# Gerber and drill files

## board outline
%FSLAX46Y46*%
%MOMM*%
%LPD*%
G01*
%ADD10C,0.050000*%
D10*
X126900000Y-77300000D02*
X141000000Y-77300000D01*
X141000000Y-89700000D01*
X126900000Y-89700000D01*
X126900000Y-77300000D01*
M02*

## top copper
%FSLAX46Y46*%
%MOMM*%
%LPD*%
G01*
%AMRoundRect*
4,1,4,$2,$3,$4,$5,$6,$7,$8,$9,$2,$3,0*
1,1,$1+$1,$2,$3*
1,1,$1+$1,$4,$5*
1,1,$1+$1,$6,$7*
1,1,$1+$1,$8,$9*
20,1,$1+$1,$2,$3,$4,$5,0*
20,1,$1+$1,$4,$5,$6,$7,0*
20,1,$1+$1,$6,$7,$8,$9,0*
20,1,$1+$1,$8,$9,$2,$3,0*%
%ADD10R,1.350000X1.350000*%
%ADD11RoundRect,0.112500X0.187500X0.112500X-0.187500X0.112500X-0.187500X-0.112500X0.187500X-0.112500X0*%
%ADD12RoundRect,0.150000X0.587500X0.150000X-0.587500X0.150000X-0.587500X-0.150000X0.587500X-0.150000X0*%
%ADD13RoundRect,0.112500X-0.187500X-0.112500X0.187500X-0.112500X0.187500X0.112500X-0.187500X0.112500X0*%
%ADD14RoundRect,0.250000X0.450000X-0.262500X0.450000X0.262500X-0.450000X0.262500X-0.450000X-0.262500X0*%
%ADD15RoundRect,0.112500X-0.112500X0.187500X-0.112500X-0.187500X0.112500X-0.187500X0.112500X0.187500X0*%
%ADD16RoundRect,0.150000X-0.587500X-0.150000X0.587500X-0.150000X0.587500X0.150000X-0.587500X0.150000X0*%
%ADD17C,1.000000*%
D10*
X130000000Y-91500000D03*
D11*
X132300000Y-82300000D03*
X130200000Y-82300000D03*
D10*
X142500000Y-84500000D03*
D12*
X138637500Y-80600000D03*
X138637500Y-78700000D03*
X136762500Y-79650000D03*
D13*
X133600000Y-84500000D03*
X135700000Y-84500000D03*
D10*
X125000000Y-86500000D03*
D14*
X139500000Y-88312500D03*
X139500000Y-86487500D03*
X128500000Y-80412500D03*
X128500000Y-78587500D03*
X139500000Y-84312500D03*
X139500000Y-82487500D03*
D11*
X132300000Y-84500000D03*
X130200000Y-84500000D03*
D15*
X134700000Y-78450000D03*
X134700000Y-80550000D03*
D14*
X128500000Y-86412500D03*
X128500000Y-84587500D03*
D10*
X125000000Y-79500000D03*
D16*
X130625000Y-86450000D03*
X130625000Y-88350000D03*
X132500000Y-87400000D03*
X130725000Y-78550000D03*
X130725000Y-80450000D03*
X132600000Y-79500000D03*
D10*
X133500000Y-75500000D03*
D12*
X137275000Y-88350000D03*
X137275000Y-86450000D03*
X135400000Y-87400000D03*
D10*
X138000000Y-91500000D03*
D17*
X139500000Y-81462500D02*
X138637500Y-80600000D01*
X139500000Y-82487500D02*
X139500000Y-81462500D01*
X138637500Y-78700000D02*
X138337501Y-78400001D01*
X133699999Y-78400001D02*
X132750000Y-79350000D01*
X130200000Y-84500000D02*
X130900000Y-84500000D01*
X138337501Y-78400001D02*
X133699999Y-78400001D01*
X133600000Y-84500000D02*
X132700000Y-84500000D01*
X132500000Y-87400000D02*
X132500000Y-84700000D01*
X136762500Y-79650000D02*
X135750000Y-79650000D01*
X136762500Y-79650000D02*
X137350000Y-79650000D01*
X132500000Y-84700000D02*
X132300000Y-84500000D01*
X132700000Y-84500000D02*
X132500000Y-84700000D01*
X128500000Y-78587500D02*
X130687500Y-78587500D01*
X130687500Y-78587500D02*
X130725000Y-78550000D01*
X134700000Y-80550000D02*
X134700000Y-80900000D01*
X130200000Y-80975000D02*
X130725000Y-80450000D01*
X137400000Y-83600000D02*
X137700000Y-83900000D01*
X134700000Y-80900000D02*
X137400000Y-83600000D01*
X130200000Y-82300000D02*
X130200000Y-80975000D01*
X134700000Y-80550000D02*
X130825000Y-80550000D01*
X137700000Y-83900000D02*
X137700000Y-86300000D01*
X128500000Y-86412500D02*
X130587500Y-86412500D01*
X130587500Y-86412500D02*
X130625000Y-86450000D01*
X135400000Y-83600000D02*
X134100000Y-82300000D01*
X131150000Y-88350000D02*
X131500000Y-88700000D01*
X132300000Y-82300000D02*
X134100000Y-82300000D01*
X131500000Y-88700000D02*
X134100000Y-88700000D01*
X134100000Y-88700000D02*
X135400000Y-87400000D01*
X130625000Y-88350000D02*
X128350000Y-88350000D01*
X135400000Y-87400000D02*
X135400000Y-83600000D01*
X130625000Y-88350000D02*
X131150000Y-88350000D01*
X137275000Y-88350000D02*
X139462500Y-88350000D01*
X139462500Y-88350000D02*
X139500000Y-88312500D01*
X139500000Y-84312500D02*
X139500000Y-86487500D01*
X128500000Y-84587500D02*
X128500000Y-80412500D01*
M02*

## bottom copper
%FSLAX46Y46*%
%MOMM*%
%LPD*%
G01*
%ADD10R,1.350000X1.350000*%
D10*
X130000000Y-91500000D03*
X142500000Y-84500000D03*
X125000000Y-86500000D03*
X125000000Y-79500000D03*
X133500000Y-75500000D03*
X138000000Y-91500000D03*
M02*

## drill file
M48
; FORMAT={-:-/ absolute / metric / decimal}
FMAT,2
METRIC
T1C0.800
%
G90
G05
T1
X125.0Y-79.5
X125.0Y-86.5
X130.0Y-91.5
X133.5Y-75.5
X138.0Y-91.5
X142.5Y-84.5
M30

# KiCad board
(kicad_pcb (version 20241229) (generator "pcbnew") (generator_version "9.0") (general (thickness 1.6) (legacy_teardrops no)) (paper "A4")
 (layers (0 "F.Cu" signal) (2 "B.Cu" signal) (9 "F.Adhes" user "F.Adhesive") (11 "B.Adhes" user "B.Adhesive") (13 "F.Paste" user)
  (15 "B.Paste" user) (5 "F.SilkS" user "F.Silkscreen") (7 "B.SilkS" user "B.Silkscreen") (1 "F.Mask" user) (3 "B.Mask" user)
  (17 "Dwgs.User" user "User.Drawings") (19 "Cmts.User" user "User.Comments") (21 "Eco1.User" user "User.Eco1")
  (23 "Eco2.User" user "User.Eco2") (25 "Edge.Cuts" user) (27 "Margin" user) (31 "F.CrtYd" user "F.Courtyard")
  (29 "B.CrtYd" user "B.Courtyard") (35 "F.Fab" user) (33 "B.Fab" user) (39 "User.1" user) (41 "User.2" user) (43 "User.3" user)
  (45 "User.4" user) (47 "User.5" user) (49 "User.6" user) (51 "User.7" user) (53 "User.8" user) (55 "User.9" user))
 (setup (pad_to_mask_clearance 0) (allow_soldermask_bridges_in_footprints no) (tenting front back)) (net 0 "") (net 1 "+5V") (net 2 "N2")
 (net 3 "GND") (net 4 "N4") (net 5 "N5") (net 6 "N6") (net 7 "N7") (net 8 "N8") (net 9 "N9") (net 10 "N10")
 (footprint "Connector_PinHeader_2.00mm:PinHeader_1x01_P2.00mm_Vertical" (layer "F.Cu") (at 130 91.5)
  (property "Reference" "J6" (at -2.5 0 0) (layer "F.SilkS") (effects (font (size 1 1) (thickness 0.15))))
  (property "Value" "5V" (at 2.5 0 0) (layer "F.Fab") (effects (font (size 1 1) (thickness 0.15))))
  (pad "1" thru_hole rect (at 0 0) (size 1.35 1.35) (drill 0.8) (layers "*.Cu" "*.Mask") (remove_unused_layers no) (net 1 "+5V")))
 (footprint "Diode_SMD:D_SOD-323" (layer "F.Cu") (at 131.25 82.3 180)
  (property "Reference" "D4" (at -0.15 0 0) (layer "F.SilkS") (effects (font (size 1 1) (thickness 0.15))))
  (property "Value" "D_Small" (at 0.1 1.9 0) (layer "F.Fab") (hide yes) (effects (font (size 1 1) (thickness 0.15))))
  (pad "1" smd roundrect (at -1.05 0 180) (size 0.6 0.45) (layers "F.Cu" "F.Mask" "F.Paste") (roundrect_rratio 0.25) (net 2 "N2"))
  (pad "2" smd roundrect (at 1.05 0 180) (size 0.6 0.45) (layers "F.Cu" "F.Mask" "F.Paste") (roundrect_rratio 0.25) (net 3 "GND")))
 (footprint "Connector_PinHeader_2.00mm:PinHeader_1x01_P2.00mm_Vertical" (layer "F.Cu") (at 142.5 84.5)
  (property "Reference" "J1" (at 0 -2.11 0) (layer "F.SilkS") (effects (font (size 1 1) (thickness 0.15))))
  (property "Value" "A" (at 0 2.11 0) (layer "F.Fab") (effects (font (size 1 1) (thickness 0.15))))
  (pad "1" thru_hole rect (at 0 0) (size 1.35 1.35) (drill 0.8) (layers "*.Cu" "*.Mask") (remove_unused_layers no) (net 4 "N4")))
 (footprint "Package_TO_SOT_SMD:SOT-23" (layer "F.Cu") (at 137.7 79.65 180)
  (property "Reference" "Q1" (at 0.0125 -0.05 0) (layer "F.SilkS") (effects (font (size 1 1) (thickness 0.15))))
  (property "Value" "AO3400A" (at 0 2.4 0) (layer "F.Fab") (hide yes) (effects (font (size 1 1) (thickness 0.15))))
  (pad "1" smd roundrect (at -0.9375 -0.95 180) (size 1.475 0.6) (layers "F.Cu" "F.Mask" "F.Paste") (roundrect_rratio 0.25) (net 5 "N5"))
  (pad "2" smd roundrect (at -0.9375 0.95 180) (size 1.475 0.6) (layers "F.Cu" "F.Mask" "F.Paste") (roundrect_rratio 0.25) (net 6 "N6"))
  (pad "3" smd roundrect (at 0.9375 0 180) (size 1.475 0.6) (layers "F.Cu" "F.Mask" "F.Paste") (roundrect_rratio 0.25) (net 1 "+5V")))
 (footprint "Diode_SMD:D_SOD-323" (layer "F.Cu") (at 134.65 84.5)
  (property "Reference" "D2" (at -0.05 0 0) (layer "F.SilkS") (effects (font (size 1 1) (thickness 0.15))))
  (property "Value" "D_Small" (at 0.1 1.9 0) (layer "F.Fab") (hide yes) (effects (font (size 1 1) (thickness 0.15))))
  (pad "1" smd roundrect (at -1.05 0) (size 0.6 0.45) (layers "F.Cu" "F.Mask" "F.Paste") (roundrect_rratio 0.25) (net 1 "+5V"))
  (pad "2" smd roundrect (at 1.05 0) (size 0.6 0.45) (layers "F.Cu" "F.Mask" "F.Paste") (roundrect_rratio 0.25) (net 2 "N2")))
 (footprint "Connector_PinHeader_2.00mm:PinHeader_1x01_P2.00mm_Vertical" (layer "F.Cu") (at 125 86.5)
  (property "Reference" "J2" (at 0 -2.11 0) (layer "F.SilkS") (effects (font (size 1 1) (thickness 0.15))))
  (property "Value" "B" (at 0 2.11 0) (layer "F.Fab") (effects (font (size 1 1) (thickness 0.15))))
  (pad "1" thru_hole rect (at 0 0) (size 1.35 1.35) (drill 0.8) (layers "*.Cu" "*.Mask") (remove_unused_layers no) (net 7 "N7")))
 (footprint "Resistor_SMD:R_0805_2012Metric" (layer "F.Cu") (at 139.5 87.4 90)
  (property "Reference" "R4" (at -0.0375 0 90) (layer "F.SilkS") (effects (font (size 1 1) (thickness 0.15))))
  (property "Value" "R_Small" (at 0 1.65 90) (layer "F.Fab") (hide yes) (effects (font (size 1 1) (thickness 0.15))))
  (pad "1" smd roundrect (at -0.9125 0 90) (size 1.025 1.4) (layers "F.Cu" "F.Mask" "F.Paste") (roundrect_rratio 0.243902) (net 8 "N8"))
  (pad "2" smd roundrect (at 0.9125 0 90) (size 1.025 1.4) (layers "F.Cu" "F.Mask" "F.Paste") (roundrect_rratio 0.243902) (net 4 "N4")))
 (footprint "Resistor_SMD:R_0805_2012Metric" (layer "F.Cu") (at 128.5 79.5 90)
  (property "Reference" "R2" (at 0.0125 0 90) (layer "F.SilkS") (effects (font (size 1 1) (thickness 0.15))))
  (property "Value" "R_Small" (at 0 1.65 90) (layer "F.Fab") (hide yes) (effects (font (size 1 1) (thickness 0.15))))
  (pad "1" smd roundrect (at -0.9125 0 90) (size 1.025 1.4) (layers "F.Cu" "F.Mask" "F.Paste") (roundrect_rratio 0.243902) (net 7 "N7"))
  (pad "2" smd roundrect (at 0.9125 0 90) (size 1.025 1.4) (layers "F.Cu" "F.Mask" "F.Paste") (roundrect_rratio 0.243902) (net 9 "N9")))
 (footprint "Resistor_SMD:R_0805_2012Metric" (layer "F.Cu") (at 139.5 83.4 90)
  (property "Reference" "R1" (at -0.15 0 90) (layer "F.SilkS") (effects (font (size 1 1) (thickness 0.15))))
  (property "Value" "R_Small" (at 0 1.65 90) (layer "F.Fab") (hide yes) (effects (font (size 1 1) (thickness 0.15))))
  (pad "1" smd roundrect (at -0.9125 0 90) (size 1.025 1.4) (layers "F.Cu" "F.Mask" "F.Paste") (roundrect_rratio 0.243902) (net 4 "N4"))
  (pad "2" smd roundrect (at 0.9125 0 90) (size 1.025 1.4) (layers "F.Cu" "F.Mask" "F.Paste") (roundrect_rratio 0.243902) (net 5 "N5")))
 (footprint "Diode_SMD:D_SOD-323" (layer "F.Cu") (at 131.25 84.5 180)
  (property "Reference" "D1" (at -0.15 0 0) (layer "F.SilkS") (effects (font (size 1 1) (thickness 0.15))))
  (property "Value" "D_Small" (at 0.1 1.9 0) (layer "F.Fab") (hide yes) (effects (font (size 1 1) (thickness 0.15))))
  (pad "1" smd roundrect (at -1.05 0 180) (size 0.6 0.45) (layers "F.Cu" "F.Mask" "F.Paste") (roundrect_rratio 0.25) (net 1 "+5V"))
  (pad "2" smd roundrect (at 1.05 0 180) (size 0.6 0.45) (layers "F.Cu" "F.Mask" "F.Paste") (roundrect_rratio 0.25) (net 6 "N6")))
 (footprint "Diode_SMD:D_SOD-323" (layer "F.Cu") (at 134.7 79.5 -90)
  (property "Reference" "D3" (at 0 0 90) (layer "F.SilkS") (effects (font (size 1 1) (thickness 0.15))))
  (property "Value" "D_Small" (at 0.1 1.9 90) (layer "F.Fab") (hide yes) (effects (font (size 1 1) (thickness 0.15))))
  (pad "1" smd roundrect (at -1.05 0 270) (size 0.6 0.45) (layers "F.Cu" "F.Mask" "F.Paste") (roundrect_rratio 0.25) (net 6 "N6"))
  (pad "2" smd roundrect (at 1.05 0 270) (size 0.6 0.45) (layers "F.Cu" "F.Mask" "F.Paste") (roundrect_rratio 0.25) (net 3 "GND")))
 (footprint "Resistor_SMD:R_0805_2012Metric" (layer "F.Cu") (at 128.5 85.5 90)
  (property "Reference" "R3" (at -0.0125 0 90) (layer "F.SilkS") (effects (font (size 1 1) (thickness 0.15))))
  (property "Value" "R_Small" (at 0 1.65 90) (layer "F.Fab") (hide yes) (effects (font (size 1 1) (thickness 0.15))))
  (pad "1" smd roundrect (at -0.9125 0 90) (size 1.025 1.4) (layers "F.Cu" "F.Mask" "F.Paste") (roundrect_rratio 0.243902) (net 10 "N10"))
  (pad "2" smd roundrect (at 0.9125 0 90) (size 1.025 1.4) (layers "F.Cu" "F.Mask" "F.Paste") (roundrect_rratio 0.243902) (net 7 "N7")))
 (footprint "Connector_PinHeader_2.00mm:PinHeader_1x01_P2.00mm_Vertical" (layer "F.Cu") (at 125 79.5)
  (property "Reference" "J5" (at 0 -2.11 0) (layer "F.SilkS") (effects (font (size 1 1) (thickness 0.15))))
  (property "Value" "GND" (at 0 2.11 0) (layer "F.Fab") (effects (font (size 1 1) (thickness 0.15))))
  (pad "1" thru_hole rect (at 0 0) (size 1.35 1.35) (drill 0.8) (layers "*.Cu" "*.Mask") (remove_unused_layers no) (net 3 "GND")))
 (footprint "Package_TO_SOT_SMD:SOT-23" (layer "F.Cu") (at 131.5625 87.4)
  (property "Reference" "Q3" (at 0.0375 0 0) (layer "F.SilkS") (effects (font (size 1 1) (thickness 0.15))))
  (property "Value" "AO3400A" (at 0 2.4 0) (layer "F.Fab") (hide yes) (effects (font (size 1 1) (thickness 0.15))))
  (pad "1" smd roundrect (at -0.9375 -0.95) (size 1.475 0.6) (layers "F.Cu" "F.Mask" "F.Paste") (roundrect_rratio 0.25) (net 10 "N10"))
  (pad "2" smd roundrect (at -0.9375 0.95) (size 1.475 0.6) (layers "F.Cu" "F.Mask" "F.Paste") (roundrect_rratio 0.25) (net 2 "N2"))
  (pad "3" smd roundrect (at 0.9375 0) (size 1.475 0.6) (layers "F.Cu" "F.Mask" "F.Paste") (roundrect_rratio 0.25) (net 1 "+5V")))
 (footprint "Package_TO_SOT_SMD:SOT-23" (layer "F.Cu") (at 131.6625 79.5)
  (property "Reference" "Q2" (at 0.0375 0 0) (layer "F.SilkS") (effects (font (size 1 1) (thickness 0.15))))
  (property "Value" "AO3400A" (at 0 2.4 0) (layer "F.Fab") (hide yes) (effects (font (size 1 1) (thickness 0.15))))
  (pad "1" smd roundrect (at -0.9375 -0.95) (size 1.475 0.6) (layers "F.Cu" "F.Mask" "F.Paste") (roundrect_rratio 0.25) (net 9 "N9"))
  (pad "2" smd roundrect (at -0.9375 0.95) (size 1.475 0.6) (layers "F.Cu" "F.Mask" "F.Paste") (roundrect_rratio 0.25) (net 3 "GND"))
  (pad "3" smd roundrect (at 0.9375 0) (size 1.475 0.6) (layers "F.Cu" "F.Mask" "F.Paste") (roundrect_rratio 0.25) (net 6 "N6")))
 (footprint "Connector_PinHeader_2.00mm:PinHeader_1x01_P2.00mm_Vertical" (layer "F.Cu") (at 133.5 75.5)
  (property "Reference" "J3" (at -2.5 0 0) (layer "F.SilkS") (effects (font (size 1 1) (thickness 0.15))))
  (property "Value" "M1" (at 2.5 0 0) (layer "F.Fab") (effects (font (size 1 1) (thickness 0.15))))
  (pad "1" thru_hole rect (at 0 0) (size 1.35 1.35) (drill 0.8) (layers "*.Cu" "*.Mask") (remove_unused_layers no) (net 6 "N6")))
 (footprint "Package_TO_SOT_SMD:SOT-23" (layer "F.Cu") (at 136.3375 87.4 180)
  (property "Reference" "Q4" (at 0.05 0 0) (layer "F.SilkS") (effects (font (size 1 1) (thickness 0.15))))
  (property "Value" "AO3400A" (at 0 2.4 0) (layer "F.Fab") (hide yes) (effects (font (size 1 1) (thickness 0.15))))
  (pad "1" smd roundrect (at -0.9375 -0.95 180) (size 1.475 0.6) (layers "F.Cu" "F.Mask" "F.Paste") (roundrect_rratio 0.25) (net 8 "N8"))
  (pad "2" smd roundrect (at -0.9375 0.95 180) (size 1.475 0.6) (layers "F.Cu" "F.Mask" "F.Paste") (roundrect_rratio 0.25) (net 3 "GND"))
  (pad "3" smd roundrect (at 0.9375 0 180) (size 1.475 0.6) (layers "F.Cu" "F.Mask" "F.Paste") (roundrect_rratio 0.25) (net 2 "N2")))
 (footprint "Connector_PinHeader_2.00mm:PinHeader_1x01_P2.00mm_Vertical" (layer "F.Cu") (at 138 91.5)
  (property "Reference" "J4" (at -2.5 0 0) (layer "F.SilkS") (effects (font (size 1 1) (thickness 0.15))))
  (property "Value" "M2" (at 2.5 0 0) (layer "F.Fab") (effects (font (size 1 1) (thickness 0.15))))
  (pad "1" thru_hole rect (at 0 0) (size 1.35 1.35) (drill 0.8) (layers "*.Cu" "*.Mask") (remove_unused_layers no) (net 2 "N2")))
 (gr_rect (start 126.9 77.3) (end 141 89.7) (stroke (width 0.05) (type default)) (fill no) (layer "Edge.Cuts"))
 (segment (start 139.5 81.4625) (end 138.6375 80.6) (width 1) (layer "F.Cu") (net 5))
 (segment (start 139.5 82.4875) (end 139.5 81.4625) (width 1) (layer "F.Cu") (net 5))
 (segment (start 138.6375 78.7) (end 138.337501 78.400001) (width 1) (layer "F.Cu") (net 6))
 (segment (start 133.699999 78.400001) (end 132.75 79.35) (width 1) (layer "F.Cu") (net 6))
 (segment (start 130.2 84.5) (end 130.9 84.5) (width 1) (layer "F.Cu") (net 6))
 (segment (start 138.337501 78.400001) (end 133.699999 78.400001) (width 1) (layer "F.Cu") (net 6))
 (segment (start 133.6 84.5) (end 132.7 84.5) (width 1) (layer "F.Cu") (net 1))
 (segment (start 132.5 87.4) (end 132.5 84.7) (width 1) (layer "F.Cu") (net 1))
 (segment (start 136.7625 79.65) (end 135.75 79.65) (width 1) (layer "F.Cu") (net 1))
 (segment (start 136.7625 79.65) (end 137.35 79.65) (width 1) (layer "F.Cu") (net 1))
 (segment (start 132.5 84.7) (end 132.3 84.5) (width 1) (layer "F.Cu") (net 1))
 (segment (start 132.7 84.5) (end 132.5 84.7) (width 1) (layer "F.Cu") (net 1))
 (segment (start 128.5 78.5875) (end 130.6875 78.5875) (width 1) (layer "F.Cu") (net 9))
 (segment (start 130.6875 78.5875) (end 130.725 78.55) (width 1) (layer "F.Cu") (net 9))
 (segment (start 134.7 80.55) (end 134.7 80.9) (width 1) (layer "F.Cu") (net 3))
 (segment (start 130.2 80.975) (end 130.725 80.45) (width 1) (layer "F.Cu") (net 3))
 (segment (start 137.4 83.6) (end 137.7 83.9) (width 1) (layer "F.Cu") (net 3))
 (segment (start 134.7 80.9) (end 137.4 83.6) (width 1) (layer "F.Cu") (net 3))
 (segment (start 130.2 82.3) (end 130.2 80.975) (width 1) (layer "F.Cu") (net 3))
 (segment (start 134.7 80.55) (end 130.825 80.55) (width 1) (layer "F.Cu") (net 3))
 (segment (start 137.7 83.9) (end 137.7 86.3) (width 1) (layer "F.Cu") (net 3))
 (segment (start 128.5 86.4125) (end 130.5875 86.4125) (width 1) (layer "F.Cu") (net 10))
 (segment (start 130.5875 86.4125) (end 130.625 86.45) (width 1) (layer "F.Cu") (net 10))
 (segment (start 135.4 83.6) (end 134.1 82.3) (width 1) (layer "F.Cu") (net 2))
 (segment (start 131.15 88.35) (end 131.5 88.7) (width 1) (layer "F.Cu") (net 2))
 (segment (start 132.3 82.3) (end 134.1 82.3) (width 1) (layer "F.Cu") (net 2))
 (segment (start 131.5 88.7) (end 134.1 88.7) (width 1) (layer "F.Cu") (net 2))
 (segment (start 134.1 88.7) (end 135.4 87.4) (width 1) (layer "F.Cu") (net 2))
 (segment (start 130.625 88.35) (end 128.35 88.35) (width 1) (layer "F.Cu") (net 2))
 (segment (start 135.4 87.4) (end 135.4 83.6) (width 1) (layer "F.Cu") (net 2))
 (segment (start 130.625 88.35) (end 131.15 88.35) (width 1) (layer "F.Cu") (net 2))
 (segment (start 137.275 88.35) (end 139.4625 88.35) (width 1) (layer "F.Cu") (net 8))
 (segment (start 139.4625 88.35) (end 139.5 88.3125) (width 1) (layer "F.Cu") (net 8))
 (segment (start 139.5 84.3125) (end 139.5 86.4875) (width 1) (layer "F.Cu") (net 4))
 (segment (start 128.5 84.5875) (end 128.5 80.4125) (width 1) (layer "F.Cu") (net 7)))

